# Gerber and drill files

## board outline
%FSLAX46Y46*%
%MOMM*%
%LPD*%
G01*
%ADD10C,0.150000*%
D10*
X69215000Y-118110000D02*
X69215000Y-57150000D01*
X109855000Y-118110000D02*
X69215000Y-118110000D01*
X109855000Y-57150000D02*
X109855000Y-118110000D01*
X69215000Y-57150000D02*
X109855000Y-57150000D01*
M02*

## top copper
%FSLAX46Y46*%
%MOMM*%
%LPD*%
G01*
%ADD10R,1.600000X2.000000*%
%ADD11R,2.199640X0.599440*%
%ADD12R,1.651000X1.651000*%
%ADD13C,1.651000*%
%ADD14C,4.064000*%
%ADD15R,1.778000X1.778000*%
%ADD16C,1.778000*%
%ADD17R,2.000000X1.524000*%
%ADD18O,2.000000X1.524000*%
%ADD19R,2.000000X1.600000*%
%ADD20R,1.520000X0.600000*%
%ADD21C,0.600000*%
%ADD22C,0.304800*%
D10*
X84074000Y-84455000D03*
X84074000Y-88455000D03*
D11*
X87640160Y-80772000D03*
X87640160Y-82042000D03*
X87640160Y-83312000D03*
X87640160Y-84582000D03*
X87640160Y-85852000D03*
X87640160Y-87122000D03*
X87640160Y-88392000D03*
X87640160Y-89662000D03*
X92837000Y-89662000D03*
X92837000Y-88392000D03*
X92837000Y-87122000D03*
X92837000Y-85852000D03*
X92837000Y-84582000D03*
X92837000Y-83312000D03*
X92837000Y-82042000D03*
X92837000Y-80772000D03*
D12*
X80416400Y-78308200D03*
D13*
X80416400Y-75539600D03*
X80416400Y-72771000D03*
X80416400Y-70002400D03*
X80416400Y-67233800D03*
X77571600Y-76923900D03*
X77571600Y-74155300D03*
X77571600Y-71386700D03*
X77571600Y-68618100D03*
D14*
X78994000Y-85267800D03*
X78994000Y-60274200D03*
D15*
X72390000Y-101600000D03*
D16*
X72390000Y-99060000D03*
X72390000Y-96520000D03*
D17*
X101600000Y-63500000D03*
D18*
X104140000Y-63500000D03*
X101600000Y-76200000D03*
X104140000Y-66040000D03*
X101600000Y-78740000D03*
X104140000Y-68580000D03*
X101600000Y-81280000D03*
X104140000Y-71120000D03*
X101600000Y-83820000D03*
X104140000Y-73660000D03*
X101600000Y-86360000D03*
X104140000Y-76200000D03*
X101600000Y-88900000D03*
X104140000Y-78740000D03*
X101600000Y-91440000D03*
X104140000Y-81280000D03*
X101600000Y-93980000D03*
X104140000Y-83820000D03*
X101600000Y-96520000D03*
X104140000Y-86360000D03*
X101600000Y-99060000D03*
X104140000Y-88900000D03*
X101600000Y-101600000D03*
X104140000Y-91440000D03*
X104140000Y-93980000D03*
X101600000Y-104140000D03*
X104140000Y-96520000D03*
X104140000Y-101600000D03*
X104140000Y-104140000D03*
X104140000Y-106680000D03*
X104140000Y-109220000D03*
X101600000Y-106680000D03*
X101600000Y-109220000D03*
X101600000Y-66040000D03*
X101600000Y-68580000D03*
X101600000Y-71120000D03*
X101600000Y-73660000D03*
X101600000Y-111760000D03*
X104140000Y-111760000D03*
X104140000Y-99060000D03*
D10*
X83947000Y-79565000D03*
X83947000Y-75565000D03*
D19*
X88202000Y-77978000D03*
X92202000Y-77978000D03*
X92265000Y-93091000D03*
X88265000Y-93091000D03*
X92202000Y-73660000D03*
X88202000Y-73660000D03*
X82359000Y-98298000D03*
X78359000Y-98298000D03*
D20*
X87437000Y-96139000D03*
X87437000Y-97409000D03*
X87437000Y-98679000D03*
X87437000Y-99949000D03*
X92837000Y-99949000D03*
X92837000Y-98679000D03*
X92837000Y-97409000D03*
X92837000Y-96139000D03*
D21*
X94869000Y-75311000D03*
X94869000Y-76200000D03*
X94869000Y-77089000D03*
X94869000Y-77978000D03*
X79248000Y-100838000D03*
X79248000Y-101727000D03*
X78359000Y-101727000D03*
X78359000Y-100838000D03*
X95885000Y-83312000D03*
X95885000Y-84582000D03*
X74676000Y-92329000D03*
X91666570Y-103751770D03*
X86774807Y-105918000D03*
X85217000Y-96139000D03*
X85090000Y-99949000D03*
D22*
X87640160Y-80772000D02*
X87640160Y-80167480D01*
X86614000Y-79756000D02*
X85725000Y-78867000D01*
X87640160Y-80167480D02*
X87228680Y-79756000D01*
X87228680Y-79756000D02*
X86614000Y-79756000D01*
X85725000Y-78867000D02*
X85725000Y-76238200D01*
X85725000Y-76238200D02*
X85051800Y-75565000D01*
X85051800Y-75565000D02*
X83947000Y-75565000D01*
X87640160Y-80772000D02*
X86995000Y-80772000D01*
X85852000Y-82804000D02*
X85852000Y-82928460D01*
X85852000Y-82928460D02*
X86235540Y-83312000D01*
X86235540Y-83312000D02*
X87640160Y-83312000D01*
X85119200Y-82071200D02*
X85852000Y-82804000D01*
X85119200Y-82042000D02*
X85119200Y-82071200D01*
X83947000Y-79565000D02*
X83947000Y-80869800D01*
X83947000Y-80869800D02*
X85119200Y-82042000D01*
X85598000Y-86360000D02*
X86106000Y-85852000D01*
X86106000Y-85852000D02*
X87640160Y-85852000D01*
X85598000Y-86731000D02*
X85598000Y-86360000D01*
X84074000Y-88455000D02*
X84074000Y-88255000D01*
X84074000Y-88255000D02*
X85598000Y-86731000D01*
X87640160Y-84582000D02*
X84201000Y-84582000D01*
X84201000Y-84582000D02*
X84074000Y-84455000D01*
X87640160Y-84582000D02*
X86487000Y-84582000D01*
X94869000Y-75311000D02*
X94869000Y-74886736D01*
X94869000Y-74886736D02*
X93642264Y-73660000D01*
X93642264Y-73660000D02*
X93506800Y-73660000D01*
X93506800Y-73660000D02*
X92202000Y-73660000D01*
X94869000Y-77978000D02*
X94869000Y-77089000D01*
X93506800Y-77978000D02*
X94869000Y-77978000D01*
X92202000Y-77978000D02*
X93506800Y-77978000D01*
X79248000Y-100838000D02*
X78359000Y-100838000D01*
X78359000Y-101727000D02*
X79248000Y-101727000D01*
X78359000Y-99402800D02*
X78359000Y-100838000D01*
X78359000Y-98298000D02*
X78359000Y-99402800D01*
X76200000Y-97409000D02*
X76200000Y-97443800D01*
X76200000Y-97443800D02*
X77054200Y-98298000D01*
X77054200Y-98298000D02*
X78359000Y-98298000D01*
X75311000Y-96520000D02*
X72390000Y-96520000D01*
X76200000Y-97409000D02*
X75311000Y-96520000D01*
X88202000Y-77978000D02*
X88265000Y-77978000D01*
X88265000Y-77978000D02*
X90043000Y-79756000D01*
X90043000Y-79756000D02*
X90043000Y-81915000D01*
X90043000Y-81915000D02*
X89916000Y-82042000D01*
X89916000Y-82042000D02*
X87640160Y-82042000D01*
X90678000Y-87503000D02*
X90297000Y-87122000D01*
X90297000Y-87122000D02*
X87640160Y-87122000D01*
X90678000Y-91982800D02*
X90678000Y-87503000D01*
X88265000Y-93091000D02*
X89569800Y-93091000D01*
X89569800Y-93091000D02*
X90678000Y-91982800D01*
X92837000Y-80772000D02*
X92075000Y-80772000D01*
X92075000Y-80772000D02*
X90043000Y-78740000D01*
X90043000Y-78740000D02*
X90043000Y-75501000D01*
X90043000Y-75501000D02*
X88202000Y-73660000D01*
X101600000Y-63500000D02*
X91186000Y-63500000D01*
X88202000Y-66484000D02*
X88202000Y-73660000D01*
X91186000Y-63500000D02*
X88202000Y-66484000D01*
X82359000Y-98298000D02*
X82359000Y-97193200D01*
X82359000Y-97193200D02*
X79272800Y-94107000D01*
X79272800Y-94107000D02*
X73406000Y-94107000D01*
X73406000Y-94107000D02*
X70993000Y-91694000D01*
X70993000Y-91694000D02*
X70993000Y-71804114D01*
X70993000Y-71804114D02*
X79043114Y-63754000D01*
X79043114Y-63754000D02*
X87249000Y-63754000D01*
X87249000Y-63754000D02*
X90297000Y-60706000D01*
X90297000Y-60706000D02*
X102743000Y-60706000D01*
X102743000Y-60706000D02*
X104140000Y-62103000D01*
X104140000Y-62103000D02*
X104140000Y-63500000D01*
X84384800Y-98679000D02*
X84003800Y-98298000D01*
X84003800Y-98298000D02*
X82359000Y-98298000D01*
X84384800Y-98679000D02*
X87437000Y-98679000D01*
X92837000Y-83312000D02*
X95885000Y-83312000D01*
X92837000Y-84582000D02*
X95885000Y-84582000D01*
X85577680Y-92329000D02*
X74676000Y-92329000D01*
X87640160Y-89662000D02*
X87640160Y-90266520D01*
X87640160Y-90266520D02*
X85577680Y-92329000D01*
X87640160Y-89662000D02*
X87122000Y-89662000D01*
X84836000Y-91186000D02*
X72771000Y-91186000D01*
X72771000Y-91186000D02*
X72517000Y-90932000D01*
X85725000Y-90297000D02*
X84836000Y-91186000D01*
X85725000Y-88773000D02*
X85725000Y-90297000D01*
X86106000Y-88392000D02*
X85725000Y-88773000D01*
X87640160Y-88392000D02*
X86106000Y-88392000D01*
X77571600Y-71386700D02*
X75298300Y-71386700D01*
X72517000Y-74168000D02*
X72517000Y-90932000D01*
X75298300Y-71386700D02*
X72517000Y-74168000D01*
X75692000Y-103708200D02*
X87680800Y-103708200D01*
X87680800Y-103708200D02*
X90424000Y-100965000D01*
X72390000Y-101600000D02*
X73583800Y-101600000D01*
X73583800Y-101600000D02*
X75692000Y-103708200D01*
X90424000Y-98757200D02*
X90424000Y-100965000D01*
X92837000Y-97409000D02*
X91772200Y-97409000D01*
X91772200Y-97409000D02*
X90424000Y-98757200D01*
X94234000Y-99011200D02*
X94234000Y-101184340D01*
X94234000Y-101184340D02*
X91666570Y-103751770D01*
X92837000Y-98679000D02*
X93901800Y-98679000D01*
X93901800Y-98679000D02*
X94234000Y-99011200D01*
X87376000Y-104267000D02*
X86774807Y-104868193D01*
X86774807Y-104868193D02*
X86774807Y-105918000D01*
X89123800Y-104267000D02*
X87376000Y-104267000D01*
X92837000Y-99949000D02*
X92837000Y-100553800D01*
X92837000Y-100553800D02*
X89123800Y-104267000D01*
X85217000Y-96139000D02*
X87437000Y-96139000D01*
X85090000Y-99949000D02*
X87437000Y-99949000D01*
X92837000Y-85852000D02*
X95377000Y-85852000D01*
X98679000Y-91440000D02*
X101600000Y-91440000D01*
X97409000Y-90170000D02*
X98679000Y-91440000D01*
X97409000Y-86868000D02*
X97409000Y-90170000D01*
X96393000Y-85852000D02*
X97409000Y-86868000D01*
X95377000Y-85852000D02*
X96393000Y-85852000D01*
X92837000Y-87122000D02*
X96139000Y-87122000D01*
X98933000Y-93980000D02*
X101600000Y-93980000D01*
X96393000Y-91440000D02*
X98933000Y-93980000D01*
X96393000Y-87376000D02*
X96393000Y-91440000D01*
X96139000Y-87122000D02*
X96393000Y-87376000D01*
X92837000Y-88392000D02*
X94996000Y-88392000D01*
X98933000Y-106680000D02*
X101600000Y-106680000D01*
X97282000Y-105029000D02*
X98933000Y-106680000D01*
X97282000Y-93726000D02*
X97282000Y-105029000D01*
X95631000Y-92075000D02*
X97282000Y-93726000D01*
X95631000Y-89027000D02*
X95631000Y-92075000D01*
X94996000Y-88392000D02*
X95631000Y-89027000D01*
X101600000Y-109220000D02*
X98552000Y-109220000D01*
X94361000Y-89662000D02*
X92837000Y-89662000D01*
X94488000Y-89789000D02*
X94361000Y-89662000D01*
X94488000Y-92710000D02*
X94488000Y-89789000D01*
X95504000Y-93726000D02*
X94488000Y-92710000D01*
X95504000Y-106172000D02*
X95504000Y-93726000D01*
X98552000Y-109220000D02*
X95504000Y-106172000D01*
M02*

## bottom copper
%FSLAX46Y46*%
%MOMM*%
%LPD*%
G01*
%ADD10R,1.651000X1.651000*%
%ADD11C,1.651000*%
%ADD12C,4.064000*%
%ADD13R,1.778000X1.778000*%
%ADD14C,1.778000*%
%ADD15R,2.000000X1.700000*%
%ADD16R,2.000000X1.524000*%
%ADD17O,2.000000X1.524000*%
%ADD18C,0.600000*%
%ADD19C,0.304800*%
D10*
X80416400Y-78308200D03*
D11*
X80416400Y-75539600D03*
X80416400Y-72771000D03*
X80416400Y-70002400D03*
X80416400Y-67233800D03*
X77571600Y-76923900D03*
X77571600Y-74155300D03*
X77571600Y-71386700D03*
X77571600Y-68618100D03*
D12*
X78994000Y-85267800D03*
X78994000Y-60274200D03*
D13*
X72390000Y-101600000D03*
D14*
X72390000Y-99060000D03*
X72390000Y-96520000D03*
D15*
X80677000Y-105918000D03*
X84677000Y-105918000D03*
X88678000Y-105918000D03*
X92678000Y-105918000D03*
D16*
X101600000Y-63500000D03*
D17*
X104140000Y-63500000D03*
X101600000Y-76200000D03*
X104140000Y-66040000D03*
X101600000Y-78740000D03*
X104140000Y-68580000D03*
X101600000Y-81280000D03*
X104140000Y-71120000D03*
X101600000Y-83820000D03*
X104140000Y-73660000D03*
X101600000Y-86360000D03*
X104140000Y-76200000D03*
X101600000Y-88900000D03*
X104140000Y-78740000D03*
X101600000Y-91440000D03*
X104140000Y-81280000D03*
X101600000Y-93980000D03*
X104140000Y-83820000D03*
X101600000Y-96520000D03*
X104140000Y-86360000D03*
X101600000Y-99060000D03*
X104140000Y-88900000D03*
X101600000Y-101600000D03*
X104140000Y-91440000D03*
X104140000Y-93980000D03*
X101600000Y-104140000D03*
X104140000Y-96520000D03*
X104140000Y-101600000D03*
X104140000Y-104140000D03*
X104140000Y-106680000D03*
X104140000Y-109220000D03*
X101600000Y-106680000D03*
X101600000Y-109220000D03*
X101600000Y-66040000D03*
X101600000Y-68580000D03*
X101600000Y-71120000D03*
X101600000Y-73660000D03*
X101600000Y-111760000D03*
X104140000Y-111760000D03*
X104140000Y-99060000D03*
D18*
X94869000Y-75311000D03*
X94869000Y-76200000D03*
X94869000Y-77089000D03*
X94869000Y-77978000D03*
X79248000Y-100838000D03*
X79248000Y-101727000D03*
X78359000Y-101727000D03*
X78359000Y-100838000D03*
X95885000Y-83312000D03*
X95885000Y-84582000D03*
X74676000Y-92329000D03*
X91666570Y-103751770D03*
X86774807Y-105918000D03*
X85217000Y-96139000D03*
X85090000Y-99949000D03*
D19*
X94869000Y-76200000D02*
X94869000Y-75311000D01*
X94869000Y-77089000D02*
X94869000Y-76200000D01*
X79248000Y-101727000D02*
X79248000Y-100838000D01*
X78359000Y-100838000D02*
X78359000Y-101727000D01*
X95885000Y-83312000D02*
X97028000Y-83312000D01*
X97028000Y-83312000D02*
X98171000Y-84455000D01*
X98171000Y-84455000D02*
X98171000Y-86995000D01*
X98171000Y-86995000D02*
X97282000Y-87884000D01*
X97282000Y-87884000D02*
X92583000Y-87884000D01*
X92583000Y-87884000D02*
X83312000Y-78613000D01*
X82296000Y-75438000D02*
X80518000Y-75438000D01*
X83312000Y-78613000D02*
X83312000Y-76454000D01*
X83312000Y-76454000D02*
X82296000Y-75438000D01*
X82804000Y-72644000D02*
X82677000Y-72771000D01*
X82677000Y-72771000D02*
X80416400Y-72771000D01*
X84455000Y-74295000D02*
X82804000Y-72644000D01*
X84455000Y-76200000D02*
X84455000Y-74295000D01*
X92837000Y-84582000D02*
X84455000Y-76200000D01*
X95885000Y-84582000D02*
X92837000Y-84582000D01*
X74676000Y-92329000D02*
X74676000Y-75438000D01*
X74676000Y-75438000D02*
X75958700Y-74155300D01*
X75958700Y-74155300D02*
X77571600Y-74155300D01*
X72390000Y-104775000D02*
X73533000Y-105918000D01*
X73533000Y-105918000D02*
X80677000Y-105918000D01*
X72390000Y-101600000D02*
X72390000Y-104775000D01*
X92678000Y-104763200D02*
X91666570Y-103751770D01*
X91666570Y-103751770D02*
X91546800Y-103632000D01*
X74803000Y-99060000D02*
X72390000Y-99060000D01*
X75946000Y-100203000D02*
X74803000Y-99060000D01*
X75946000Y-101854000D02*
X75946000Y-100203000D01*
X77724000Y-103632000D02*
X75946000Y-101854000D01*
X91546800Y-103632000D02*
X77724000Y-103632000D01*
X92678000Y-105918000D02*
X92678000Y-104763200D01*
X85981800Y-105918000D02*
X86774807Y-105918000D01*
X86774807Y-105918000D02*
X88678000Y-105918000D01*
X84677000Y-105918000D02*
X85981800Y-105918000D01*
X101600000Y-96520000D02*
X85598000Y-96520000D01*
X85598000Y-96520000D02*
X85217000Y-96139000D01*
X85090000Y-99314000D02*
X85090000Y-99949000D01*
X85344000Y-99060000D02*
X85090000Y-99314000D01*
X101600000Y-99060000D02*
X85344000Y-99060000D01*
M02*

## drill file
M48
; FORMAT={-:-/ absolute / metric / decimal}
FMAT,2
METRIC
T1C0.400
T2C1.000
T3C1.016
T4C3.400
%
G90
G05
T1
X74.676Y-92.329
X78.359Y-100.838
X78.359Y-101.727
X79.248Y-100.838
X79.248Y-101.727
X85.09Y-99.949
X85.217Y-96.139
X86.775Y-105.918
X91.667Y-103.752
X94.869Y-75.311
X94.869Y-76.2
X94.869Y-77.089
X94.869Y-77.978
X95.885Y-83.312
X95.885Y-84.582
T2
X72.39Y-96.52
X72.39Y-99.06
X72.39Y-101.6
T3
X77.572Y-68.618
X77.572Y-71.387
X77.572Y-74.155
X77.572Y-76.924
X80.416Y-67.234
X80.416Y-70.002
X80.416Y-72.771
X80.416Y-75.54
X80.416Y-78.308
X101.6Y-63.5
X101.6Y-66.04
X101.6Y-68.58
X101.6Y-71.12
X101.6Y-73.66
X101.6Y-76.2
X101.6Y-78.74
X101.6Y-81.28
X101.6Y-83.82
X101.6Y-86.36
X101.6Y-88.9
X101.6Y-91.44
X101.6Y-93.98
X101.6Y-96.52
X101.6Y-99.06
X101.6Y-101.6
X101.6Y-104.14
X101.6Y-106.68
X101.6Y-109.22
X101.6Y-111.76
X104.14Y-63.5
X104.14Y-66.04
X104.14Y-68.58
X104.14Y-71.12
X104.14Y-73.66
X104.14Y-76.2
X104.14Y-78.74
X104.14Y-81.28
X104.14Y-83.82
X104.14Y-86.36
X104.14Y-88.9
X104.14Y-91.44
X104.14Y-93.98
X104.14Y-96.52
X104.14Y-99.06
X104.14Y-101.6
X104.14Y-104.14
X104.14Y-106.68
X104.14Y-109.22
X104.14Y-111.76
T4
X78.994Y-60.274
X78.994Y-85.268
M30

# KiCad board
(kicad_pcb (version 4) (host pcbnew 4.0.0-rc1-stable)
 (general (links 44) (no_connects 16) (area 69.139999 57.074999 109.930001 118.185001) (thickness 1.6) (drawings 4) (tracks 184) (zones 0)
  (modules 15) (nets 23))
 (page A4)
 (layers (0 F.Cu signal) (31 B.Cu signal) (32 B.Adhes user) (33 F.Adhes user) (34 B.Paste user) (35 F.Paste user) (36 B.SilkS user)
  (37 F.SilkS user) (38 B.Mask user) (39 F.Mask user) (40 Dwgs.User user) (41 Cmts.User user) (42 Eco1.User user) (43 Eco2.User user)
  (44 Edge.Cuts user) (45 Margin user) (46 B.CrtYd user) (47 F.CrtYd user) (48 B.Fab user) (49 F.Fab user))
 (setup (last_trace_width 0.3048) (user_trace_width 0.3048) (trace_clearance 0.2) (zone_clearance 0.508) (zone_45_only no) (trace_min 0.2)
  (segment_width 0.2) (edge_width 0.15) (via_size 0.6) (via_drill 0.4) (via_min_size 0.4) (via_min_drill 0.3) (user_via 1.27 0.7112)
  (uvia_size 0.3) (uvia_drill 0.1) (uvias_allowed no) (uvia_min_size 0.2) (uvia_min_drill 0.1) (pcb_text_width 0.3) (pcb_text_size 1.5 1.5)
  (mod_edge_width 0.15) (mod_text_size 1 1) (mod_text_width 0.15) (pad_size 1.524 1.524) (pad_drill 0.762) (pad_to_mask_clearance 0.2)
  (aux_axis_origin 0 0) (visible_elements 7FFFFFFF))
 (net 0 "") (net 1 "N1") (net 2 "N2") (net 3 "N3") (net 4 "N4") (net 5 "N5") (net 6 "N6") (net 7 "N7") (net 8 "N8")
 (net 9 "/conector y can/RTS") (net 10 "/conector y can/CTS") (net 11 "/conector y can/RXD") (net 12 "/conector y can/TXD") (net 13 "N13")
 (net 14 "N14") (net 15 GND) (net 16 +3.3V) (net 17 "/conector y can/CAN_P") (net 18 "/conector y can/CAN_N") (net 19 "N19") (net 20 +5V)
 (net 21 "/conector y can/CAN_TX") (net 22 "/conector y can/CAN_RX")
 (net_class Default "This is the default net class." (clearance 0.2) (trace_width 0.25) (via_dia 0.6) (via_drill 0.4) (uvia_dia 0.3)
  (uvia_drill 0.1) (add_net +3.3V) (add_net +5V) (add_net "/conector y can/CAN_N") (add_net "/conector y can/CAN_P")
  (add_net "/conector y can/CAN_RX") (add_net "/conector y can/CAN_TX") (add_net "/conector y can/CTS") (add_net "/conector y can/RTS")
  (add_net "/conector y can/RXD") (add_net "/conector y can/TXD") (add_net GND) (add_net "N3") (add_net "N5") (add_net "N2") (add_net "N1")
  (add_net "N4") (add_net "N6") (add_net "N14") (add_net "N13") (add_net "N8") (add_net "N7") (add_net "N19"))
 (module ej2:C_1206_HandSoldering (layer F.Cu) (at 84.074 86.455 90)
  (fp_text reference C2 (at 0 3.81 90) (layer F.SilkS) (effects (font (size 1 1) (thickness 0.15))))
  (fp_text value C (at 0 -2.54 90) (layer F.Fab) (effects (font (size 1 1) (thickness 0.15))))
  (pad 2 smd rect (at 2 0 90) (size 2 1.6) (layers F.Cu F.Paste F.Mask) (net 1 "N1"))
  (pad 1 smd rect (at -2 0 90) (size 2 1.6) (layers F.Cu F.Paste F.Mask) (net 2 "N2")))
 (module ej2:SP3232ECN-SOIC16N (layer F.Cu) (at 90.23858 85.217 270)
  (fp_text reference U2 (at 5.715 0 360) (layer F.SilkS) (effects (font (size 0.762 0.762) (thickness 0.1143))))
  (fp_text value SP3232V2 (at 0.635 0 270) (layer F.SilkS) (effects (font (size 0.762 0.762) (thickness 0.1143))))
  (pad 1 smd rect (at -4.445 2.59842 270) (size 0.59944 2.19964) (layers F.Cu F.Paste F.Mask) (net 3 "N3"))
  (pad 2 smd rect (at -3.175 2.59842 270) (size 0.59944 2.19964) (layers F.Cu F.Paste F.Mask) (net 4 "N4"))
  (pad 3 smd rect (at -1.905 2.59842 270) (size 0.59944 2.19964) (layers F.Cu F.Paste F.Mask) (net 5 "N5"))
  (pad 4 smd rect (at -0.635 2.59842 270) (size 0.59944 2.19964) (layers F.Cu F.Paste F.Mask) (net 1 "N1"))
  (pad 5 smd rect (at 0.635 2.59842 270) (size 0.59944 2.19964) (layers F.Cu F.Paste F.Mask) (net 2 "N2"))
  (pad 6 smd rect (at 1.905 2.59842 270) (size 0.59944 2.19964) (layers F.Cu F.Paste F.Mask) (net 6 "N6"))
  (pad 7 smd rect (at 3.175 2.59842 270) (size 0.59944 2.19964) (layers F.Cu F.Paste F.Mask) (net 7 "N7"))
  (pad 8 smd rect (at 4.445 2.59842 270) (size 0.59944 2.19964) (layers F.Cu F.Paste F.Mask) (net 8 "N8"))
  (pad 9 smd rect (at 4.445 -2.59842 270) (size 0.59944 2.19964) (layers F.Cu F.Paste F.Mask) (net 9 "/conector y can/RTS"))
  (pad 10 smd rect (at 3.175 -2.59842 270) (size 0.59944 2.19964) (layers F.Cu F.Paste F.Mask) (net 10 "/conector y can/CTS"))
  (pad 11 smd rect (at 1.905 -2.59842 270) (size 0.59944 2.19964) (layers F.Cu F.Paste F.Mask) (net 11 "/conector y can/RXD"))
  (pad 12 smd rect (at 0.635 -2.59842 270) (size 0.59944 2.19964) (layers F.Cu F.Paste F.Mask) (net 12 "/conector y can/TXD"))
  (pad 13 smd rect (at -0.635 -2.59842 270) (size 0.59944 2.19964) (layers F.Cu F.Paste F.Mask) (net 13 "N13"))
  (pad 14 smd rect (at -1.905 -2.59842 270) (size 0.59944 2.19964) (layers F.Cu F.Paste F.Mask) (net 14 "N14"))
  (pad 15 smd rect (at -3.175 -2.59842 270) (size 0.59944 2.19964) (layers F.Cu F.Paste F.Mask) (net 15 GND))
  (pad 16 smd rect (at -4.445 -2.59842 270) (size 0.59944 2.19964) (layers F.Cu F.Paste F.Mask) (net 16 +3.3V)))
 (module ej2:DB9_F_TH (layer F.Cu) (at 78.994 72.771 90)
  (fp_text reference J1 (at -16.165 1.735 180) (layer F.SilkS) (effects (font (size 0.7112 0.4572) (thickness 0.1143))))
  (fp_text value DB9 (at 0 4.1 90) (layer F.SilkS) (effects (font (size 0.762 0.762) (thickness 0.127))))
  (pad 1 thru_hole rect (at -5.5372 1.4224 90) (size 1.651 1.651) (drill 1.016) (layers *.Cu *.Mask))
  (pad 2 thru_hole circle (at -2.7686 1.4224 90) (size 1.651 1.651) (drill 1.016) (layers *.Cu *.Mask) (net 14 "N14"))
  (pad 3 thru_hole circle (at 0 1.4224 90) (size 1.651 1.651) (drill 1.016) (layers *.Cu *.Mask) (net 13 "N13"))
  (pad 4 thru_hole circle (at 2.7686 1.4224 90) (size 1.651 1.651) (drill 1.016) (layers *.Cu *.Mask))
  (pad 5 thru_hole circle (at 5.5372 1.4224 90) (size 1.651 1.651) (drill 1.016) (layers *.Cu *.Mask) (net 15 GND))
  (pad 6 thru_hole circle (at -4.1529 -1.4224 90) (size 1.651 1.651) (drill 1.016) (layers *.Cu *.Mask))
  (pad 7 thru_hole circle (at -1.3843 -1.4224 90) (size 1.651 1.651) (drill 1.016) (layers *.Cu *.Mask) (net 8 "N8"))
  (pad 8 thru_hole circle (at 1.3843 -1.4224 90) (size 1.651 1.651) (drill 1.016) (layers *.Cu *.Mask) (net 7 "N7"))
  (pad 9 thru_hole circle (at 4.1529 -1.4224 90) (size 1.651 1.651) (drill 1.016) (layers *.Cu *.Mask))
  (pad 10 thru_hole circle (at -12.4968 0 90) (size 4.064 4.064) (drill 3.4) (layers *.Cu *.Mask))
  (pad 11 thru_hole circle (at 12.4968 0 90) (size 4.064 4.064) (drill 3.4) (layers *.Cu *.Mask)))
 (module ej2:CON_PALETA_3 (layer F.Cu) (at 72.39 99.06 90)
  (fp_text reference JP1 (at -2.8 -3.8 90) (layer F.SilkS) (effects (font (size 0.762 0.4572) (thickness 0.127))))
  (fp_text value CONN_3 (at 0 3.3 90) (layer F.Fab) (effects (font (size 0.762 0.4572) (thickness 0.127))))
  (pad 1 thru_hole rect (at -2.54 0 90) (size 1.778 1.778) (drill 1) (layers *.Cu *.Mask) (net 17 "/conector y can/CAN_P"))
  (pad 2 thru_hole circle (at 0 0 90) (size 1.778 1.778) (drill 1) (layers *.Cu *.Mask) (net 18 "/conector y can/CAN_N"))
  (pad 3 thru_hole circle (at 2.54 0 90) (size 1.778 1.778) (drill 1) (layers *.Cu *.Mask) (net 15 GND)))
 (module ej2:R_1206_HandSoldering (layer B.Cu) (at 82.677 105.918)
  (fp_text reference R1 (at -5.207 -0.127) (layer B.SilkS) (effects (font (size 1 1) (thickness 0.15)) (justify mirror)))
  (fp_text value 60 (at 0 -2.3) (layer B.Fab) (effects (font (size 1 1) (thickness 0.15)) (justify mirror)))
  (pad 1 smd rect (at -2 0) (size 2 1.7) (layers B.Cu B.Paste B.Mask) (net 17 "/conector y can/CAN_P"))
  (pad 2 smd rect (at 2 0) (size 2 1.7) (layers B.Cu B.Paste B.Mask) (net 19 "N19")))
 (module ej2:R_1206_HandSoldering (layer B.Cu) (at 90.678 105.918)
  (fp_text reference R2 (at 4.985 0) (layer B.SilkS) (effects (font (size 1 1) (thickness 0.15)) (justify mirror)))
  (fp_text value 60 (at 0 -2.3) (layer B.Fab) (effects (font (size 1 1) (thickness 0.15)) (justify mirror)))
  (pad 1 smd rect (at -2 0) (size 2 1.7) (layers B.Cu B.Paste B.Mask) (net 19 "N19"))
  (pad 2 smd rect (at 2 0) (size 2 1.7) (layers B.Cu B.Paste B.Mask) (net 18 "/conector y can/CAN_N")))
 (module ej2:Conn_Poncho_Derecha (layer F.Cu) (at 101.6 63.5)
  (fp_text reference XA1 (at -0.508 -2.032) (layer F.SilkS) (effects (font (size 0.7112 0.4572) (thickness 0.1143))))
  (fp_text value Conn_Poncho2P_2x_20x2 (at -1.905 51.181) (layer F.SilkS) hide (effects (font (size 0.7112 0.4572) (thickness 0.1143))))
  (pad 1 thru_hole rect (at 0 0 270) (size 1.524 2) (drill 1.016) (layers *.Cu *.Mask) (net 16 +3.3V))
  (pad 2 thru_hole oval (at 2.54 0 270) (size 1.524 2) (drill 1.016) (layers *.Cu *.Mask) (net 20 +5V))
  (pad 11 thru_hole oval (at 0 12.7 270) (size 1.524 2) (drill 1.016) (layers *.Cu *.Mask))
  (pad 4 thru_hole oval (at 2.54 2.54 270) (size 1.524 2) (drill 1.016) (layers *.Cu *.Mask) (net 15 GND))
  (pad 13 thru_hole oval (at 0 15.24 270) (size 1.524 2) (drill 1.016) (layers *.Cu *.Mask))
  (pad 6 thru_hole oval (at 2.54 5.08 270) (size 1.524 2) (drill 1.016) (layers *.Cu *.Mask))
  (pad 15 thru_hole oval (at 0 17.78 270) (size 1.524 2) (drill 1.016) (layers *.Cu *.Mask))
  (pad 8 thru_hole oval (at 2.54 7.62 270) (size 1.524 2) (drill 1.016) (layers *.Cu *.Mask))
  (pad 17 thru_hole oval (at 0 20.32 270) (size 1.524 2) (drill 1.016) (layers *.Cu *.Mask))
  (pad 10 thru_hole oval (at 2.54 10.16 270) (size 1.524 2) (drill 1.016) (layers *.Cu *.Mask))
  (pad 19 thru_hole oval (at 0 22.86 270) (size 1.524 2) (drill 1.016) (layers *.Cu *.Mask))
  (pad 12 thru_hole oval (at 2.54 12.7 270) (size 1.524 2) (drill 1.016) (layers *.Cu *.Mask))
  (pad 21 thru_hole oval (at 0 25.4 270) (size 1.524 2) (drill 1.016) (layers *.Cu *.Mask))
  (pad 14 thru_hole oval (at 2.54 15.24 270) (size 1.524 2) (drill 1.016) (layers *.Cu *.Mask))
  (pad 23 thru_hole oval (at 0 27.94 270) (size 1.524 2) (drill 1.016) (layers *.Cu *.Mask) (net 12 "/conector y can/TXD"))
  (pad 16 thru_hole oval (at 2.54 17.78 270) (size 1.524 2) (drill 1.016) (layers *.Cu *.Mask))
  (pad 25 thru_hole oval (at 0 30.48 270) (size 1.524 2) (drill 1.016) (layers *.Cu *.Mask) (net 11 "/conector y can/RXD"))
  (pad 18 thru_hole oval (at 2.54 20.32 270) (size 1.524 2) (drill 1.016) (layers *.Cu *.Mask))
  (pad 27 thru_hole oval (at 0 33.02 270) (size 1.524 2) (drill 1.016) (layers *.Cu *.Mask) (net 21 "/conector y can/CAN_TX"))
  (pad 20 thru_hole oval (at 2.54 22.86 270) (size 1.524 2) (drill 1.016) (layers *.Cu *.Mask) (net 15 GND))
  (pad 29 thru_hole oval (at 0 35.56 270) (size 1.524 2) (drill 1.016) (layers *.Cu *.Mask) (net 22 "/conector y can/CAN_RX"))
  (pad 22 thru_hole oval (at 2.54 25.4 270) (size 1.524 2) (drill 1.016) (layers *.Cu *.Mask) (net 15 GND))
  (pad 31 thru_hole oval (at 0 38.1 270) (size 1.524 2) (drill 1.016) (layers *.Cu *.Mask))
  (pad 24 thru_hole oval (at 2.54 27.94 270) (size 1.524 2) (drill 1.016) (layers *.Cu *.Mask) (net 15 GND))
  (pad 26 thru_hole oval (at 2.54 30.48 270) (size 1.524 2) (drill 1.016) (layers *.Cu *.Mask) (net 15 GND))
  (pad 33 thru_hole oval (at 0 40.64 270) (size 1.524 2) (drill 1.016) (layers *.Cu *.Mask))
  (pad 28 thru_hole oval (at 2.54 33.02 270) (size 1.524 2) (drill 1.016) (layers *.Cu *.Mask) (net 15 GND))
  (pad 32 thru_hole oval (at 2.54 38.1 270) (size 1.524 2) (drill 1.016) (layers *.Cu *.Mask) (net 15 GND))
  (pad 34 thru_hole oval (at 2.54 40.64 270) (size 1.524 2) (drill 1.016) (layers *.Cu *.Mask))
  (pad 36 thru_hole oval (at 2.54 43.18 270) (size 1.524 2) (drill 1.016) (layers *.Cu *.Mask))
  (pad 38 thru_hole oval (at 2.54 45.72 270) (size 1.524 2) (drill 1.016) (layers *.Cu *.Mask) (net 15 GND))
  (pad 35 thru_hole oval (at 0 43.18 270) (size 1.524 2) (drill 1.016) (layers *.Cu *.Mask) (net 10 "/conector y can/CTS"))
  (pad 37 thru_hole oval (at 0 45.72 270) (size 1.524 2) (drill 1.016) (layers *.Cu *.Mask) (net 9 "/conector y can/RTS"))
  (pad 3 thru_hole oval (at 0 2.54 270) (size 1.524 2) (drill 1.016) (layers *.Cu *.Mask))
  (pad 5 thru_hole oval (at 0 5.08 270) (size 1.524 2) (drill 1.016) (layers *.Cu *.Mask))
  (pad 7 thru_hole oval (at 0 7.62 270) (size 1.524 2) (drill 1.016) (layers *.Cu *.Mask))
  (pad 9 thru_hole oval (at 0 10.16 270) (size 1.524 2) (drill 1.016) (layers *.Cu *.Mask))
  (pad 39 thru_hole oval (at 0 48.26 270) (size 1.524 2) (drill 1.016) (layers *.Cu *.Mask))
  (pad 40 thru_hole oval (at 2.54 48.26 270) (size 1.524 2) (drill 1.016) (layers *.Cu *.Mask) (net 15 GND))
  (pad 30 thru_hole oval (at 2.54 35.56 270) (size 1.524 2) (drill 1.016) (layers *.Cu *.Mask) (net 15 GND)))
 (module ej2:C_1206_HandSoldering (layer F.Cu) (at 83.947 77.565 270)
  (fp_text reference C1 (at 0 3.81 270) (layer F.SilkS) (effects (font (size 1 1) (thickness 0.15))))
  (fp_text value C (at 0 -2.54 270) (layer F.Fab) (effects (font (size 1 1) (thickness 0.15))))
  (pad 2 smd rect (at 2 0 270) (size 2 1.6) (layers F.Cu F.Paste F.Mask) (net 5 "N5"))
  (pad 1 smd rect (at -2 0 270) (size 2 1.6) (layers F.Cu F.Paste F.Mask) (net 3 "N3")))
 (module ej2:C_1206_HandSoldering (layer F.Cu) (at 90.202 77.978 180)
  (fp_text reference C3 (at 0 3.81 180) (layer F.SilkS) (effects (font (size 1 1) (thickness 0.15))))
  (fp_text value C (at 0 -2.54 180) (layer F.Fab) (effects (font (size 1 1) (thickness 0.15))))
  (pad 2 smd rect (at 2 0 180) (size 2 1.6) (layers F.Cu F.Paste F.Mask) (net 4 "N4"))
  (pad 1 smd rect (at -2 0 180) (size 2 1.6) (layers F.Cu F.Paste F.Mask) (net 15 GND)))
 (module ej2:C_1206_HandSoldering (layer F.Cu) (at 90.265 93.091)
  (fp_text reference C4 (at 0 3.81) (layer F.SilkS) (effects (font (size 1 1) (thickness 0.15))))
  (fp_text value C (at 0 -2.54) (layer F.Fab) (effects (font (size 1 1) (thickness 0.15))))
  (pad 2 smd rect (at 2 0) (size 2 1.6) (layers F.Cu F.Paste F.Mask) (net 15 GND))
  (pad 1 smd rect (at -2 0) (size 2 1.6) (layers F.Cu F.Paste F.Mask) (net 6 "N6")))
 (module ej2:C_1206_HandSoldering (layer F.Cu) (at 90.202 73.66)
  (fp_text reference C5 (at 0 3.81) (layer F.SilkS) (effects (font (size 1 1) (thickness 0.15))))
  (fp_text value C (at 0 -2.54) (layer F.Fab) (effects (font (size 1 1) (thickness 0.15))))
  (pad 2 smd rect (at 2 0) (size 2 1.6) (layers F.Cu F.Paste F.Mask) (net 15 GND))
  (pad 1 smd rect (at -2 0) (size 2 1.6) (layers F.Cu F.Paste F.Mask) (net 16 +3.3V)))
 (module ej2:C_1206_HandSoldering (layer F.Cu) (at 80.359 98.298)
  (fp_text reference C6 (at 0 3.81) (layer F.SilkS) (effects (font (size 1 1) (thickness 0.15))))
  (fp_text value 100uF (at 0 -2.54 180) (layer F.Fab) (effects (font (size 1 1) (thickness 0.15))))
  (pad 2 smd rect (at 2 0) (size 2 1.6) (layers F.Cu F.Paste F.Mask) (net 20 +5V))
  (pad 1 smd rect (at -2 0) (size 2 1.6) (layers F.Cu F.Paste F.Mask) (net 15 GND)))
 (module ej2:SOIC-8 (layer F.Cu) (at 90.137 98.044)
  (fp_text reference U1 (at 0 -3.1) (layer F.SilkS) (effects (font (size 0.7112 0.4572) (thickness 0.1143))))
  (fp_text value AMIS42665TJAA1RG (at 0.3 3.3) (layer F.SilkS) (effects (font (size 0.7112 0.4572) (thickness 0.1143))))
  (pad 1 smd rect (at -2.7 -1.905 270) (size 0.6 1.52) (layers F.Cu F.Paste F.Mask) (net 21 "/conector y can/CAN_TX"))
  (pad 2 smd rect (at -2.7 -0.635 270) (size 0.6 1.52) (layers F.Cu F.Paste F.Mask) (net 15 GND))
  (pad 3 smd rect (at -2.7 0.635 270) (size 0.6 1.52) (layers F.Cu F.Paste F.Mask) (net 20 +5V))
  (pad 4 smd rect (at -2.7 1.905 270) (size 0.6 1.52) (layers F.Cu F.Paste F.Mask) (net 22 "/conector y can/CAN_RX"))
  (pad 5 smd rect (at 2.7 1.905 270) (size 0.6 1.52) (layers F.Cu F.Paste F.Mask) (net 19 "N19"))
  (pad 6 smd rect (at 2.7 0.635 270) (size 0.6 1.52) (layers F.Cu F.Paste F.Mask) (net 18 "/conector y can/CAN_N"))
  (pad 7 smd rect (at 2.7 -0.635 270) (size 0.6 1.52) (layers F.Cu F.Paste F.Mask) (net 17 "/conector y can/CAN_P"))
  (pad 8 smd rect (at 2.7 -1.905 270) (size 0.6 1.52) (layers F.Cu F.Paste F.Mask) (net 15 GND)))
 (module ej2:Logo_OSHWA (layer F.Cu) (at 89.916 63.881)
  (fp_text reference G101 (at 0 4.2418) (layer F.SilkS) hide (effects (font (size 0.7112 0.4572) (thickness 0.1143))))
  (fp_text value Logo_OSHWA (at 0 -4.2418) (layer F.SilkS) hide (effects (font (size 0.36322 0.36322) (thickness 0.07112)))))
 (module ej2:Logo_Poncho (layer F.Cu) (at 87.884 108.204)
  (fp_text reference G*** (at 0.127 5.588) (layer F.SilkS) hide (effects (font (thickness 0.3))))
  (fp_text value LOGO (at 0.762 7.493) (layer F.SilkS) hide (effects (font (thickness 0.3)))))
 (gr_line (start 69.215 118.11) (end 69.215 57.15) (angle 90) (layer Edge.Cuts) (width 0.15))
 (gr_line (start 109.855 118.11) (end 69.215 118.11) (angle 90) (layer Edge.Cuts) (width 0.15))
 (gr_line (start 109.855 57.15) (end 109.855 118.11) (angle 90) (layer Edge.Cuts) (width 0.15))
 (gr_line (start 69.215 57.15) (end 109.855 57.15) (angle 90) (layer Edge.Cuts) (width 0.15))
 (segment (start 87.64016 80.772) (end 87.64016 80.16748) (width 0.3048) (layer F.Cu) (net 3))
 (segment (start 86.614 79.756) (end 85.725 78.867) (width 0.3048) (layer F.Cu) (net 3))
 (segment (start 87.64016 80.16748) (end 87.22868 79.756) (width 0.3048) (layer F.Cu) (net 3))
 (segment (start 87.22868 79.756) (end 86.614 79.756) (width 0.3048) (layer F.Cu) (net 3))
 (segment (start 85.725 78.867) (end 85.725 76.2382) (width 0.3048) (layer F.Cu) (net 3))
 (segment (start 85.725 76.2382) (end 85.0518 75.565) (width 0.3048) (layer F.Cu) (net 3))
 (segment (start 85.0518 75.565) (end 83.947 75.565) (width 0.3048) (layer F.Cu) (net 3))
 (segment (start 87.64016 80.772) (end 86.995 80.772) (width 0.3048) (layer F.Cu) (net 3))
 (segment (start 85.852 82.804) (end 85.852 82.92846) (width 0.3048) (layer F.Cu) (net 5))
 (segment (start 85.852 82.92846) (end 86.23554 83.312) (width 0.3048) (layer F.Cu) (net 5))
 (segment (start 86.23554 83.312) (end 87.64016 83.312) (width 0.3048) (layer F.Cu) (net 5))
 (segment (start 85.1192 82.0712) (end 85.852 82.804) (width 0.3048) (layer F.Cu) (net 5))
 (segment (start 85.1192 82.042) (end 85.1192 82.0712) (width 0.3048) (layer F.Cu) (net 5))
 (segment (start 83.947 79.565) (end 83.947 80.8698) (width 0.3048) (layer F.Cu) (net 5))
 (segment (start 83.947 80.8698) (end 85.1192 82.042) (width 0.3048) (layer F.Cu) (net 5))
 (segment (start 85.598 86.36) (end 86.106 85.852) (width 0.3048) (layer F.Cu) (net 2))
 (segment (start 86.106 85.852) (end 87.64016 85.852) (width 0.3048) (layer F.Cu) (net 2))
 (segment (start 85.598 86.731) (end 85.598 86.36) (width 0.3048) (layer F.Cu) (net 2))
 (segment (start 84.074 88.455) (end 84.074 88.255) (width 0.3048) (layer F.Cu) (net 2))
 (segment (start 84.074 88.255) (end 85.598 86.731) (width 0.3048) (layer F.Cu) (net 2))
 (segment (start 87.64016 84.582) (end 84.201 84.582) (width 0.3048) (layer F.Cu) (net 1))
 (segment (start 84.201 84.582) (end 84.074 84.455) (width 0.3048) (layer F.Cu) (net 1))
 (segment (start 87.64016 84.582) (end 86.487 84.582) (width 0.3048) (layer F.Cu) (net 1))
 (segment (start 94.869 75.311) (end 94.869 74.886736) (width 0.3048) (layer F.Cu) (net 15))
 (segment (start 94.869 74.886736) (end 93.642264 73.66) (width 0.3048) (layer F.Cu) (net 15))
 (segment (start 93.642264 73.66) (end 93.5068 73.66) (width 0.3048) (layer F.Cu) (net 15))
 (segment (start 93.5068 73.66) (end 92.202 73.66) (width 0.3048) (layer F.Cu) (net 15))
 (segment (start 94.869 76.2) (end 94.869 75.311) (width 0.3048) (layer B.Cu) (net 15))
 (via (at 94.869 75.311) (size 0.6) (drill 0.4) (layers F.Cu B.Cu) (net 15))
 (via (at 94.869 76.2) (size 0.6) (drill 0.4) (layers F.Cu B.Cu) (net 15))
 (segment (start 94.869 77.089) (end 94.869 76.2) (width 0.3048) (layer B.Cu) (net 15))
 (segment (start 94.869 77.978) (end 94.869 77.089) (width 0.3048) (layer F.Cu) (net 15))
 (via (at 94.869 77.089) (size 0.6) (drill 0.4) (layers F.Cu B.Cu) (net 15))
 (via (at 94.869 77.978) (size 0.6) (drill 0.4) (layers F.Cu B.Cu) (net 15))
 (segment (start 93.5068 77.978) (end 94.869 77.978) (width 0.3048) (layer F.Cu) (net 15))
 (segment (start 92.202 77.978) (end 93.5068 77.978) (width 0.3048) (layer F.Cu) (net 15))
 (segment (start 79.248 100.838) (end 78.359 100.838) (width 0.3048) (layer F.Cu) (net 15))
 (segment (start 79.248 101.727) (end 79.248 100.838) (width 0.3048) (layer B.Cu) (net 15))
 (via (at 79.248 100.838) (size 0.6) (drill 0.4) (layers F.Cu B.Cu) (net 15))
 (segment (start 78.359 101.727) (end 79.248 101.727) (width 0.3048) (layer F.Cu) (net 15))
 (via (at 79.248 101.727) (size 0.6) (drill 0.4) (layers F.Cu B.Cu) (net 15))
 (segment (start 78.359 100.838) (end 78.359 101.727) (width 0.3048) (layer B.Cu) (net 15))
 (via (at 78.359 101.727) (size 0.6) (drill 0.4) (layers F.Cu B.Cu) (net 15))
 (segment (start 78.359 99.4028) (end 78.359 100.838) (width 0.3048) (layer F.Cu) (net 15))
 (via (at 78.359 100.838) (size 0.6) (drill 0.4) (layers F.Cu B.Cu) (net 15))
 (segment (start 78.359 98.298) (end 78.359 99.4028) (width 0.3048) (layer F.Cu) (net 15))
 (segment (start 76.2 97.409) (end 76.2 97.4438) (width 0.3048) (layer F.Cu) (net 15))
 (segment (start 76.2 97.4438) (end 77.0542 98.298) (width 0.3048) (layer F.Cu) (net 15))
 (segment (start 77.0542 98.298) (end 78.359 98.298) (width 0.3048) (layer F.Cu) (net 15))
 (segment (start 75.311 96.52) (end 72.39 96.52) (width 0.3048) (layer F.Cu) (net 15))
 (segment (start 76.2 97.409) (end 75.311 96.52) (width 0.3048) (layer F.Cu) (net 15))
 (segment (start 88.202 77.978) (end 88.265 77.978) (width 0.3048) (layer F.Cu) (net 4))
 (segment (start 88.265 77.978) (end 90.043 79.756) (width 0.3048) (layer F.Cu) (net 4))
 (segment (start 90.043 79.756) (end 90.043 81.915) (width 0.3048) (layer F.Cu) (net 4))
 (segment (start 90.043 81.915) (end 89.916 82.042) (width 0.3048) (layer F.Cu) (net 4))
 (segment (start 89.916 82.042) (end 87.64016 82.042) (width 0.3048) (layer F.Cu) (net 4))
 (segment (start 90.678 87.503) (end 90.297 87.122) (width 0.3048) (layer F.Cu) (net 6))
 (segment (start 90.297 87.122) (end 87.64016 87.122) (width 0.3048) (layer F.Cu) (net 6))
 (segment (start 90.678 91.9828) (end 90.678 87.503) (width 0.3048) (layer F.Cu) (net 6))
 (segment (start 88.265 93.091) (end 89.5698 93.091) (width 0.3048) (layer F.Cu) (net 6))
 (segment (start 89.5698 93.091) (end 90.678 91.9828) (width 0.3048) (layer F.Cu) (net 6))
 (segment (start 92.837 80.772) (end 92.075 80.772) (width 0.3048) (layer F.Cu) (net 16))
 (segment (start 92.075 80.772) (end 90.043 78.74) (width 0.3048) (layer F.Cu) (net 16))
 (segment (start 90.043 78.74) (end 90.043 75.501) (width 0.3048) (layer F.Cu) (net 16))
 (segment (start 90.043 75.501) (end 88.202 73.66) (width 0.3048) (layer F.Cu) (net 16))
 (segment (start 101.6 63.5) (end 91.186 63.5) (width 0.3048) (layer F.Cu) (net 16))
 (segment (start 88.202 66.484) (end 88.202 73.66) (width 0.3048) (layer F.Cu) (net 16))
 (segment (start 91.186 63.5) (end 88.202 66.484) (width 0.3048) (layer F.Cu) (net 16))
 (segment (start 82.359 98.298) (end 82.359 97.1932) (width 0.3048) (layer F.Cu) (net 20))
 (segment (start 82.359 97.1932) (end 79.2728 94.107) (width 0.3048) (layer F.Cu) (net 20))
 (segment (start 79.2728 94.107) (end 73.406 94.107) (width 0.3048) (layer F.Cu) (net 20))
 (segment (start 73.406 94.107) (end 70.993 91.694) (width 0.3048) (layer F.Cu) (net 20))
 (segment (start 70.993 91.694) (end 70.993 71.804114) (width 0.3048) (layer F.Cu) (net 20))
 (segment (start 70.993 71.804114) (end 79.043114 63.754) (width 0.3048) (layer F.Cu) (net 20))
 (segment (start 79.043114 63.754) (end 87.249 63.754) (width 0.3048) (layer F.Cu) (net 20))
 (segment (start 87.249 63.754) (end 90.297 60.706) (width 0.3048) (layer F.Cu) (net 20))
 (segment (start 90.297 60.706) (end 102.743 60.706) (width 0.3048) (layer F.Cu) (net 20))
 (segment (start 102.743 60.706) (end 104.14 62.103) (width 0.3048) (layer F.Cu) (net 20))
 (segment (start 104.14 62.103) (end 104.14 63.5) (width 0.3048) (layer F.Cu) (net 20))
 (segment (start 84.3848 98.679) (end 84.0038 98.298) (width 0.3048) (layer F.Cu) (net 20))
 (segment (start 84.0038 98.298) (end 82.359 98.298) (width 0.3048) (layer F.Cu) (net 20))
 (segment (start 84.3848 98.679) (end 87.437 98.679) (width 0.3048) (layer F.Cu) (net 20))
 (segment (start 95.885 83.312) (end 97.028 83.312) (width 0.3048) (layer B.Cu) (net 14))
 (segment (start 97.028 83.312) (end 98.171 84.455) (width 0.3048) (layer B.Cu) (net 14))
 (segment (start 98.171 84.455) (end 98.171 86.995) (width 0.3048) (layer B.Cu) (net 14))
 (segment (start 98.171 86.995) (end 97.282 87.884) (width 0.3048) (layer B.Cu) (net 14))
 (segment (start 97.282 87.884) (end 92.583 87.884) (width 0.3048) (layer B.Cu) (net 14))
 (segment (start 92.583 87.884) (end 83.312 78.613) (width 0.3048) (layer B.Cu) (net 14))
 (segment (start 82.296 75.438) (end 80.518 75.438) (width 0.3048) (layer B.Cu) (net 14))
 (segment (start 83.312 78.613) (end 83.312 76.454) (width 0.3048) (layer B.Cu) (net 14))
 (segment (start 83.312 76.454) (end 82.296 75.438) (width 0.3048) (layer B.Cu) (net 14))
 (segment (start 92.837 83.312) (end 95.885 83.312) (width 0.3048) (layer F.Cu) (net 14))
 (via (at 95.885 83.312) (size 0.6) (drill 0.4) (layers F.Cu B.Cu) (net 14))
 (segment (start 82.804 72.644) (end 82.677 72.771) (width 0.3048) (layer B.Cu) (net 13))
 (segment (start 82.677 72.771) (end 80.4164 72.771) (width 0.3048) (layer B.Cu) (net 13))
 (segment (start 84.455 74.295) (end 82.804 72.644) (width 0.3048) (layer B.Cu) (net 13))
 (segment (start 84.455 76.2) (end 84.455 74.295) (width 0.3048) (layer B.Cu) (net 13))
 (segment (start 92.837 84.582) (end 84.455 76.2) (width 0.3048) (layer B.Cu) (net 13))
 (segment (start 95.885 84.582) (end 92.837 84.582) (width 0.3048) (layer B.Cu) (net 13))
 (segment (start 92.837 84.582) (end 95.885 84.582) (width 0.3048) (layer F.Cu) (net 13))
 (via (at 95.885 84.582) (size 0.6) (drill 0.4) (layers F.Cu B.Cu) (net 13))
 (segment (start 74.676 92.329) (end 74.676 75.438) (width 0.3048) (layer B.Cu) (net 8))
 (segment (start 74.676 75.438) (end 75.9587 74.1553) (width 0.3048) (layer B.Cu) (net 8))
 (segment (start 75.9587 74.1553) (end 77.5716 74.1553) (width 0.3048) (layer B.Cu) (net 8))
 (segment (start 85.57768 92.329) (end 74.676 92.329) (width 0.3048) (layer F.Cu) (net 8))
 (via (at 74.676 92.329) (size 0.6) (drill 0.4) (layers F.Cu B.Cu) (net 8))
 (segment (start 87.64016 89.662) (end 87.64016 90.26652) (width 0.3048) (layer F.Cu) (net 8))
 (segment (start 87.64016 90.26652) (end 85.57768 92.329) (width 0.3048) (layer F.Cu) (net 8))
 (segment (start 87.64016 89.662) (end 87.122 89.662) (width 0.3048) (layer F.Cu) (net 8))
 (segment (start 84.836 91.186) (end 72.771 91.186) (width 0.3048) (layer F.Cu) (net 7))
 (segment (start 72.771 91.186) (end 72.517 90.932) (width 0.3048) (layer F.Cu) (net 7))
 (segment (start 85.725 90.297) (end 84.836 91.186) (width 0.3048) (layer F.Cu) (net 7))
 (segment (start 85.725 88.773) (end 85.725 90.297) (width 0.3048) (layer F.Cu) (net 7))
 (segment (start 86.106 88.392) (end 85.725 88.773) (width 0.3048) (layer F.Cu) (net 7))
 (segment (start 87.64016 88.392) (end 86.106 88.392) (width 0.3048) (layer F.Cu) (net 7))
 (segment (start 77.5716 71.3867) (end 75.2983 71.3867) (width 0.3048) (layer F.Cu) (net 7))
 (segment (start 72.517 74.168) (end 72.517 90.932) (width 0.3048) (layer F.Cu) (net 7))
 (segment (start 75.2983 71.3867) (end 72.517 74.168) (width 0.3048) (layer F.Cu) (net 7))
 (segment (start 75.692 103.7082) (end 87.6808 103.7082) (width 0.3048) (layer F.Cu) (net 17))
 (segment (start 87.6808 103.7082) (end 90.424 100.965) (width 0.3048) (layer F.Cu) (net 17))
 (segment (start 72.39 101.6) (end 73.5838 101.6) (width 0.3048) (layer F.Cu) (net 17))
 (segment (start 73.5838 101.6) (end 75.692 103.7082) (width 0.3048) (layer F.Cu) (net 17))
 (segment (start 90.424 98.7572) (end 90.424 100.965) (width 0.3048) (layer F.Cu) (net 17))
 (segment (start 92.837 97.409) (end 91.7722 97.409) (width 0.3048) (layer F.Cu) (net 17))
 (segment (start 91.7722 97.409) (end 90.424 98.7572) (width 0.3048) (layer F.Cu) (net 17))
 (segment (start 72.39 104.775) (end 73.533 105.918) (width 0.3048) (layer B.Cu) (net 17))
 (segment (start 73.533 105.918) (end 80.677 105.918) (width 0.3048) (layer B.Cu) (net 17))
 (segment (start 72.39 101.6) (end 72.39 104.775) (width 0.3048) (layer B.Cu) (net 17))
 (segment (start 92.678 104.7632) (end 91.66657 103.75177) (width 0.3048) (layer B.Cu) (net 18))
 (segment (start 91.66657 103.75177) (end 91.5468 103.632) (width 0.3048) (layer B.Cu) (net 18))
 (segment (start 94.234 99.0112) (end 94.234 101.18434) (width 0.3048) (layer F.Cu) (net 18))
 (segment (start 94.234 101.18434) (end 91.66657 103.75177) (width 0.3048) (layer F.Cu) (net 18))
 (via (at 91.66657 103.75177) (size 0.6) (drill 0.4) (layers F.Cu B.Cu) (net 18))
 (segment (start 92.837 98.679) (end 93.9018 98.679) (width 0.3048) (layer F.Cu) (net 18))
 (segment (start 93.9018 98.679) (end 94.234 99.0112) (width 0.3048) (layer F.Cu) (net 18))
 (segment (start 74.803 99.06) (end 72.39 99.06) (width 0.3048) (layer B.Cu) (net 18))
 (segment (start 75.946 100.203) (end 74.803 99.06) (width 0.3048) (layer B.Cu) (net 18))
 (segment (start 75.946 101.854) (end 75.946 100.203) (width 0.3048) (layer B.Cu) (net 18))
 (segment (start 77.724 103.632) (end 75.946 101.854) (width 0.3048) (layer B.Cu) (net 18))
 (segment (start 91.5468 103.632) (end 77.724 103.632) (width 0.3048) (layer B.Cu) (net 18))
 (segment (start 92.678 105.918) (end 92.678 104.7632) (width 0.3048) (layer B.Cu) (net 18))
 (segment (start 85.9818 105.918) (end 86.774807 105.918) (width 0.3048) (layer B.Cu) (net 19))
 (segment (start 86.774807 105.918) (end 88.678 105.918) (width 0.3048) (layer B.Cu) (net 19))
 (segment (start 87.376 104.267) (end 86.774807 104.868193) (width 0.3048) (layer F.Cu) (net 19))
 (segment (start 86.774807 104.868193) (end 86.774807 105.918) (width 0.3048) (layer F.Cu) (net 19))
 (via (at 86.774807 105.918) (size 0.6) (drill 0.4) (layers F.Cu B.Cu) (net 19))
 (segment (start 89.1238 104.267) (end 87.376 104.267) (width 0.3048) (layer F.Cu) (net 19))
 (segment (start 92.837 99.949) (end 92.837 100.5538) (width 0.3048) (layer F.Cu) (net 19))
 (segment (start 92.837 100.5538) (end 89.1238 104.267) (width 0.3048) (layer F.Cu) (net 19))
 (segment (start 84.677 105.918) (end 85.9818 105.918) (width 0.3048) (layer B.Cu) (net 19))
 (segment (start 85.217 96.139) (end 87.437 96.139) (width 0.3048) (layer F.Cu) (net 21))
 (segment (start 101.6 96.52) (end 85.598 96.52) (width 0.3048) (layer B.Cu) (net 21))
 (segment (start 85.598 96.52) (end 85.217 96.139) (width 0.3048) (layer B.Cu) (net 21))
 (via (at 85.217 96.139) (size 0.6) (drill 0.4) (layers F.Cu B.Cu) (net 21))
 (segment (start 85.09 99.949) (end 87.437 99.949) (width 0.3048) (layer F.Cu) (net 22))
 (segment (start 85.09 99.314) (end 85.09 99.949) (width 0.3048) (layer B.Cu) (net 22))
 (via (at 85.09 99.949) (size 0.6) (drill 0.4) (layers F.Cu B.Cu) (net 22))
 (segment (start 85.344 99.06) (end 85.09 99.314) (width 0.3048) (layer B.Cu) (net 22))
 (segment (start 101.6 99.06) (end 85.344 99.06) (width 0.3048) (layer B.Cu) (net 22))
 (segment (start 92.837 85.852) (end 95.377 85.852) (width 0.3048) (layer F.Cu) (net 12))
 (segment (start 98.679 91.44) (end 101.6 91.44) (width 0.3048) (layer F.Cu) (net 12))
 (segment (start 97.409 90.17) (end 98.679 91.44) (width 0.3048) (layer F.Cu) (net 12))
 (segment (start 97.409 86.868) (end 97.409 90.17) (width 0.3048) (layer F.Cu) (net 12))
 (segment (start 96.393 85.852) (end 97.409 86.868) (width 0.3048) (layer F.Cu) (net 12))
 (segment (start 95.377 85.852) (end 96.393 85.852) (width 0.3048) (layer F.Cu) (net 12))
 (segment (start 92.837 87.122) (end 96.139 87.122) (width 0.3048) (layer F.Cu) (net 11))
 (segment (start 98.933 93.98) (end 101.6 93.98) (width 0.3048) (layer F.Cu) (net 11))
 (segment (start 96.393 91.44) (end 98.933 93.98) (width 0.3048) (layer F.Cu) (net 11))
 (segment (start 96.393 87.376) (end 96.393 91.44) (width 0.3048) (layer F.Cu) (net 11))
 (segment (start 96.139 87.122) (end 96.393 87.376) (width 0.3048) (layer F.Cu) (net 11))
 (segment (start 92.837 88.392) (end 94.996 88.392) (width 0.3048) (layer F.Cu) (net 10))
 (segment (start 98.933 106.68) (end 101.6 106.68) (width 0.3048) (layer F.Cu) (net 10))
 (segment (start 97.282 105.029) (end 98.933 106.68) (width 0.3048) (layer F.Cu) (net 10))
 (segment (start 97.282 93.726) (end 97.282 105.029) (width 0.3048) (layer F.Cu) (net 10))
 (segment (start 95.631 92.075) (end 97.282 93.726) (width 0.3048) (layer F.Cu) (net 10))
 (segment (start 95.631 89.027) (end 95.631 92.075) (width 0.3048) (layer F.Cu) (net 10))
 (segment (start 94.996 88.392) (end 95.631 89.027) (width 0.3048) (layer F.Cu) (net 10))
 (segment (start 101.6 109.22) (end 98.552 109.22) (width 0.3048) (layer F.Cu) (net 9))
 (segment (start 94.361 89.662) (end 92.837 89.662) (width 0.3048) (layer F.Cu) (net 9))
 (segment (start 94.488 89.789) (end 94.361 89.662) (width 0.3048) (layer F.Cu) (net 9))
 (segment (start 94.488 92.71) (end 94.488 89.789) (width 0.3048) (layer F.Cu) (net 9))
 (segment (start 95.504 93.726) (end 94.488 92.71) (width 0.3048) (layer F.Cu) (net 9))
 (segment (start 95.504 106.172) (end 95.504 93.726) (width 0.3048) (layer F.Cu) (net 9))
 (segment (start 98.552 109.22) (end 95.504 106.172) (width 0.3048) (layer F.Cu) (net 9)))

